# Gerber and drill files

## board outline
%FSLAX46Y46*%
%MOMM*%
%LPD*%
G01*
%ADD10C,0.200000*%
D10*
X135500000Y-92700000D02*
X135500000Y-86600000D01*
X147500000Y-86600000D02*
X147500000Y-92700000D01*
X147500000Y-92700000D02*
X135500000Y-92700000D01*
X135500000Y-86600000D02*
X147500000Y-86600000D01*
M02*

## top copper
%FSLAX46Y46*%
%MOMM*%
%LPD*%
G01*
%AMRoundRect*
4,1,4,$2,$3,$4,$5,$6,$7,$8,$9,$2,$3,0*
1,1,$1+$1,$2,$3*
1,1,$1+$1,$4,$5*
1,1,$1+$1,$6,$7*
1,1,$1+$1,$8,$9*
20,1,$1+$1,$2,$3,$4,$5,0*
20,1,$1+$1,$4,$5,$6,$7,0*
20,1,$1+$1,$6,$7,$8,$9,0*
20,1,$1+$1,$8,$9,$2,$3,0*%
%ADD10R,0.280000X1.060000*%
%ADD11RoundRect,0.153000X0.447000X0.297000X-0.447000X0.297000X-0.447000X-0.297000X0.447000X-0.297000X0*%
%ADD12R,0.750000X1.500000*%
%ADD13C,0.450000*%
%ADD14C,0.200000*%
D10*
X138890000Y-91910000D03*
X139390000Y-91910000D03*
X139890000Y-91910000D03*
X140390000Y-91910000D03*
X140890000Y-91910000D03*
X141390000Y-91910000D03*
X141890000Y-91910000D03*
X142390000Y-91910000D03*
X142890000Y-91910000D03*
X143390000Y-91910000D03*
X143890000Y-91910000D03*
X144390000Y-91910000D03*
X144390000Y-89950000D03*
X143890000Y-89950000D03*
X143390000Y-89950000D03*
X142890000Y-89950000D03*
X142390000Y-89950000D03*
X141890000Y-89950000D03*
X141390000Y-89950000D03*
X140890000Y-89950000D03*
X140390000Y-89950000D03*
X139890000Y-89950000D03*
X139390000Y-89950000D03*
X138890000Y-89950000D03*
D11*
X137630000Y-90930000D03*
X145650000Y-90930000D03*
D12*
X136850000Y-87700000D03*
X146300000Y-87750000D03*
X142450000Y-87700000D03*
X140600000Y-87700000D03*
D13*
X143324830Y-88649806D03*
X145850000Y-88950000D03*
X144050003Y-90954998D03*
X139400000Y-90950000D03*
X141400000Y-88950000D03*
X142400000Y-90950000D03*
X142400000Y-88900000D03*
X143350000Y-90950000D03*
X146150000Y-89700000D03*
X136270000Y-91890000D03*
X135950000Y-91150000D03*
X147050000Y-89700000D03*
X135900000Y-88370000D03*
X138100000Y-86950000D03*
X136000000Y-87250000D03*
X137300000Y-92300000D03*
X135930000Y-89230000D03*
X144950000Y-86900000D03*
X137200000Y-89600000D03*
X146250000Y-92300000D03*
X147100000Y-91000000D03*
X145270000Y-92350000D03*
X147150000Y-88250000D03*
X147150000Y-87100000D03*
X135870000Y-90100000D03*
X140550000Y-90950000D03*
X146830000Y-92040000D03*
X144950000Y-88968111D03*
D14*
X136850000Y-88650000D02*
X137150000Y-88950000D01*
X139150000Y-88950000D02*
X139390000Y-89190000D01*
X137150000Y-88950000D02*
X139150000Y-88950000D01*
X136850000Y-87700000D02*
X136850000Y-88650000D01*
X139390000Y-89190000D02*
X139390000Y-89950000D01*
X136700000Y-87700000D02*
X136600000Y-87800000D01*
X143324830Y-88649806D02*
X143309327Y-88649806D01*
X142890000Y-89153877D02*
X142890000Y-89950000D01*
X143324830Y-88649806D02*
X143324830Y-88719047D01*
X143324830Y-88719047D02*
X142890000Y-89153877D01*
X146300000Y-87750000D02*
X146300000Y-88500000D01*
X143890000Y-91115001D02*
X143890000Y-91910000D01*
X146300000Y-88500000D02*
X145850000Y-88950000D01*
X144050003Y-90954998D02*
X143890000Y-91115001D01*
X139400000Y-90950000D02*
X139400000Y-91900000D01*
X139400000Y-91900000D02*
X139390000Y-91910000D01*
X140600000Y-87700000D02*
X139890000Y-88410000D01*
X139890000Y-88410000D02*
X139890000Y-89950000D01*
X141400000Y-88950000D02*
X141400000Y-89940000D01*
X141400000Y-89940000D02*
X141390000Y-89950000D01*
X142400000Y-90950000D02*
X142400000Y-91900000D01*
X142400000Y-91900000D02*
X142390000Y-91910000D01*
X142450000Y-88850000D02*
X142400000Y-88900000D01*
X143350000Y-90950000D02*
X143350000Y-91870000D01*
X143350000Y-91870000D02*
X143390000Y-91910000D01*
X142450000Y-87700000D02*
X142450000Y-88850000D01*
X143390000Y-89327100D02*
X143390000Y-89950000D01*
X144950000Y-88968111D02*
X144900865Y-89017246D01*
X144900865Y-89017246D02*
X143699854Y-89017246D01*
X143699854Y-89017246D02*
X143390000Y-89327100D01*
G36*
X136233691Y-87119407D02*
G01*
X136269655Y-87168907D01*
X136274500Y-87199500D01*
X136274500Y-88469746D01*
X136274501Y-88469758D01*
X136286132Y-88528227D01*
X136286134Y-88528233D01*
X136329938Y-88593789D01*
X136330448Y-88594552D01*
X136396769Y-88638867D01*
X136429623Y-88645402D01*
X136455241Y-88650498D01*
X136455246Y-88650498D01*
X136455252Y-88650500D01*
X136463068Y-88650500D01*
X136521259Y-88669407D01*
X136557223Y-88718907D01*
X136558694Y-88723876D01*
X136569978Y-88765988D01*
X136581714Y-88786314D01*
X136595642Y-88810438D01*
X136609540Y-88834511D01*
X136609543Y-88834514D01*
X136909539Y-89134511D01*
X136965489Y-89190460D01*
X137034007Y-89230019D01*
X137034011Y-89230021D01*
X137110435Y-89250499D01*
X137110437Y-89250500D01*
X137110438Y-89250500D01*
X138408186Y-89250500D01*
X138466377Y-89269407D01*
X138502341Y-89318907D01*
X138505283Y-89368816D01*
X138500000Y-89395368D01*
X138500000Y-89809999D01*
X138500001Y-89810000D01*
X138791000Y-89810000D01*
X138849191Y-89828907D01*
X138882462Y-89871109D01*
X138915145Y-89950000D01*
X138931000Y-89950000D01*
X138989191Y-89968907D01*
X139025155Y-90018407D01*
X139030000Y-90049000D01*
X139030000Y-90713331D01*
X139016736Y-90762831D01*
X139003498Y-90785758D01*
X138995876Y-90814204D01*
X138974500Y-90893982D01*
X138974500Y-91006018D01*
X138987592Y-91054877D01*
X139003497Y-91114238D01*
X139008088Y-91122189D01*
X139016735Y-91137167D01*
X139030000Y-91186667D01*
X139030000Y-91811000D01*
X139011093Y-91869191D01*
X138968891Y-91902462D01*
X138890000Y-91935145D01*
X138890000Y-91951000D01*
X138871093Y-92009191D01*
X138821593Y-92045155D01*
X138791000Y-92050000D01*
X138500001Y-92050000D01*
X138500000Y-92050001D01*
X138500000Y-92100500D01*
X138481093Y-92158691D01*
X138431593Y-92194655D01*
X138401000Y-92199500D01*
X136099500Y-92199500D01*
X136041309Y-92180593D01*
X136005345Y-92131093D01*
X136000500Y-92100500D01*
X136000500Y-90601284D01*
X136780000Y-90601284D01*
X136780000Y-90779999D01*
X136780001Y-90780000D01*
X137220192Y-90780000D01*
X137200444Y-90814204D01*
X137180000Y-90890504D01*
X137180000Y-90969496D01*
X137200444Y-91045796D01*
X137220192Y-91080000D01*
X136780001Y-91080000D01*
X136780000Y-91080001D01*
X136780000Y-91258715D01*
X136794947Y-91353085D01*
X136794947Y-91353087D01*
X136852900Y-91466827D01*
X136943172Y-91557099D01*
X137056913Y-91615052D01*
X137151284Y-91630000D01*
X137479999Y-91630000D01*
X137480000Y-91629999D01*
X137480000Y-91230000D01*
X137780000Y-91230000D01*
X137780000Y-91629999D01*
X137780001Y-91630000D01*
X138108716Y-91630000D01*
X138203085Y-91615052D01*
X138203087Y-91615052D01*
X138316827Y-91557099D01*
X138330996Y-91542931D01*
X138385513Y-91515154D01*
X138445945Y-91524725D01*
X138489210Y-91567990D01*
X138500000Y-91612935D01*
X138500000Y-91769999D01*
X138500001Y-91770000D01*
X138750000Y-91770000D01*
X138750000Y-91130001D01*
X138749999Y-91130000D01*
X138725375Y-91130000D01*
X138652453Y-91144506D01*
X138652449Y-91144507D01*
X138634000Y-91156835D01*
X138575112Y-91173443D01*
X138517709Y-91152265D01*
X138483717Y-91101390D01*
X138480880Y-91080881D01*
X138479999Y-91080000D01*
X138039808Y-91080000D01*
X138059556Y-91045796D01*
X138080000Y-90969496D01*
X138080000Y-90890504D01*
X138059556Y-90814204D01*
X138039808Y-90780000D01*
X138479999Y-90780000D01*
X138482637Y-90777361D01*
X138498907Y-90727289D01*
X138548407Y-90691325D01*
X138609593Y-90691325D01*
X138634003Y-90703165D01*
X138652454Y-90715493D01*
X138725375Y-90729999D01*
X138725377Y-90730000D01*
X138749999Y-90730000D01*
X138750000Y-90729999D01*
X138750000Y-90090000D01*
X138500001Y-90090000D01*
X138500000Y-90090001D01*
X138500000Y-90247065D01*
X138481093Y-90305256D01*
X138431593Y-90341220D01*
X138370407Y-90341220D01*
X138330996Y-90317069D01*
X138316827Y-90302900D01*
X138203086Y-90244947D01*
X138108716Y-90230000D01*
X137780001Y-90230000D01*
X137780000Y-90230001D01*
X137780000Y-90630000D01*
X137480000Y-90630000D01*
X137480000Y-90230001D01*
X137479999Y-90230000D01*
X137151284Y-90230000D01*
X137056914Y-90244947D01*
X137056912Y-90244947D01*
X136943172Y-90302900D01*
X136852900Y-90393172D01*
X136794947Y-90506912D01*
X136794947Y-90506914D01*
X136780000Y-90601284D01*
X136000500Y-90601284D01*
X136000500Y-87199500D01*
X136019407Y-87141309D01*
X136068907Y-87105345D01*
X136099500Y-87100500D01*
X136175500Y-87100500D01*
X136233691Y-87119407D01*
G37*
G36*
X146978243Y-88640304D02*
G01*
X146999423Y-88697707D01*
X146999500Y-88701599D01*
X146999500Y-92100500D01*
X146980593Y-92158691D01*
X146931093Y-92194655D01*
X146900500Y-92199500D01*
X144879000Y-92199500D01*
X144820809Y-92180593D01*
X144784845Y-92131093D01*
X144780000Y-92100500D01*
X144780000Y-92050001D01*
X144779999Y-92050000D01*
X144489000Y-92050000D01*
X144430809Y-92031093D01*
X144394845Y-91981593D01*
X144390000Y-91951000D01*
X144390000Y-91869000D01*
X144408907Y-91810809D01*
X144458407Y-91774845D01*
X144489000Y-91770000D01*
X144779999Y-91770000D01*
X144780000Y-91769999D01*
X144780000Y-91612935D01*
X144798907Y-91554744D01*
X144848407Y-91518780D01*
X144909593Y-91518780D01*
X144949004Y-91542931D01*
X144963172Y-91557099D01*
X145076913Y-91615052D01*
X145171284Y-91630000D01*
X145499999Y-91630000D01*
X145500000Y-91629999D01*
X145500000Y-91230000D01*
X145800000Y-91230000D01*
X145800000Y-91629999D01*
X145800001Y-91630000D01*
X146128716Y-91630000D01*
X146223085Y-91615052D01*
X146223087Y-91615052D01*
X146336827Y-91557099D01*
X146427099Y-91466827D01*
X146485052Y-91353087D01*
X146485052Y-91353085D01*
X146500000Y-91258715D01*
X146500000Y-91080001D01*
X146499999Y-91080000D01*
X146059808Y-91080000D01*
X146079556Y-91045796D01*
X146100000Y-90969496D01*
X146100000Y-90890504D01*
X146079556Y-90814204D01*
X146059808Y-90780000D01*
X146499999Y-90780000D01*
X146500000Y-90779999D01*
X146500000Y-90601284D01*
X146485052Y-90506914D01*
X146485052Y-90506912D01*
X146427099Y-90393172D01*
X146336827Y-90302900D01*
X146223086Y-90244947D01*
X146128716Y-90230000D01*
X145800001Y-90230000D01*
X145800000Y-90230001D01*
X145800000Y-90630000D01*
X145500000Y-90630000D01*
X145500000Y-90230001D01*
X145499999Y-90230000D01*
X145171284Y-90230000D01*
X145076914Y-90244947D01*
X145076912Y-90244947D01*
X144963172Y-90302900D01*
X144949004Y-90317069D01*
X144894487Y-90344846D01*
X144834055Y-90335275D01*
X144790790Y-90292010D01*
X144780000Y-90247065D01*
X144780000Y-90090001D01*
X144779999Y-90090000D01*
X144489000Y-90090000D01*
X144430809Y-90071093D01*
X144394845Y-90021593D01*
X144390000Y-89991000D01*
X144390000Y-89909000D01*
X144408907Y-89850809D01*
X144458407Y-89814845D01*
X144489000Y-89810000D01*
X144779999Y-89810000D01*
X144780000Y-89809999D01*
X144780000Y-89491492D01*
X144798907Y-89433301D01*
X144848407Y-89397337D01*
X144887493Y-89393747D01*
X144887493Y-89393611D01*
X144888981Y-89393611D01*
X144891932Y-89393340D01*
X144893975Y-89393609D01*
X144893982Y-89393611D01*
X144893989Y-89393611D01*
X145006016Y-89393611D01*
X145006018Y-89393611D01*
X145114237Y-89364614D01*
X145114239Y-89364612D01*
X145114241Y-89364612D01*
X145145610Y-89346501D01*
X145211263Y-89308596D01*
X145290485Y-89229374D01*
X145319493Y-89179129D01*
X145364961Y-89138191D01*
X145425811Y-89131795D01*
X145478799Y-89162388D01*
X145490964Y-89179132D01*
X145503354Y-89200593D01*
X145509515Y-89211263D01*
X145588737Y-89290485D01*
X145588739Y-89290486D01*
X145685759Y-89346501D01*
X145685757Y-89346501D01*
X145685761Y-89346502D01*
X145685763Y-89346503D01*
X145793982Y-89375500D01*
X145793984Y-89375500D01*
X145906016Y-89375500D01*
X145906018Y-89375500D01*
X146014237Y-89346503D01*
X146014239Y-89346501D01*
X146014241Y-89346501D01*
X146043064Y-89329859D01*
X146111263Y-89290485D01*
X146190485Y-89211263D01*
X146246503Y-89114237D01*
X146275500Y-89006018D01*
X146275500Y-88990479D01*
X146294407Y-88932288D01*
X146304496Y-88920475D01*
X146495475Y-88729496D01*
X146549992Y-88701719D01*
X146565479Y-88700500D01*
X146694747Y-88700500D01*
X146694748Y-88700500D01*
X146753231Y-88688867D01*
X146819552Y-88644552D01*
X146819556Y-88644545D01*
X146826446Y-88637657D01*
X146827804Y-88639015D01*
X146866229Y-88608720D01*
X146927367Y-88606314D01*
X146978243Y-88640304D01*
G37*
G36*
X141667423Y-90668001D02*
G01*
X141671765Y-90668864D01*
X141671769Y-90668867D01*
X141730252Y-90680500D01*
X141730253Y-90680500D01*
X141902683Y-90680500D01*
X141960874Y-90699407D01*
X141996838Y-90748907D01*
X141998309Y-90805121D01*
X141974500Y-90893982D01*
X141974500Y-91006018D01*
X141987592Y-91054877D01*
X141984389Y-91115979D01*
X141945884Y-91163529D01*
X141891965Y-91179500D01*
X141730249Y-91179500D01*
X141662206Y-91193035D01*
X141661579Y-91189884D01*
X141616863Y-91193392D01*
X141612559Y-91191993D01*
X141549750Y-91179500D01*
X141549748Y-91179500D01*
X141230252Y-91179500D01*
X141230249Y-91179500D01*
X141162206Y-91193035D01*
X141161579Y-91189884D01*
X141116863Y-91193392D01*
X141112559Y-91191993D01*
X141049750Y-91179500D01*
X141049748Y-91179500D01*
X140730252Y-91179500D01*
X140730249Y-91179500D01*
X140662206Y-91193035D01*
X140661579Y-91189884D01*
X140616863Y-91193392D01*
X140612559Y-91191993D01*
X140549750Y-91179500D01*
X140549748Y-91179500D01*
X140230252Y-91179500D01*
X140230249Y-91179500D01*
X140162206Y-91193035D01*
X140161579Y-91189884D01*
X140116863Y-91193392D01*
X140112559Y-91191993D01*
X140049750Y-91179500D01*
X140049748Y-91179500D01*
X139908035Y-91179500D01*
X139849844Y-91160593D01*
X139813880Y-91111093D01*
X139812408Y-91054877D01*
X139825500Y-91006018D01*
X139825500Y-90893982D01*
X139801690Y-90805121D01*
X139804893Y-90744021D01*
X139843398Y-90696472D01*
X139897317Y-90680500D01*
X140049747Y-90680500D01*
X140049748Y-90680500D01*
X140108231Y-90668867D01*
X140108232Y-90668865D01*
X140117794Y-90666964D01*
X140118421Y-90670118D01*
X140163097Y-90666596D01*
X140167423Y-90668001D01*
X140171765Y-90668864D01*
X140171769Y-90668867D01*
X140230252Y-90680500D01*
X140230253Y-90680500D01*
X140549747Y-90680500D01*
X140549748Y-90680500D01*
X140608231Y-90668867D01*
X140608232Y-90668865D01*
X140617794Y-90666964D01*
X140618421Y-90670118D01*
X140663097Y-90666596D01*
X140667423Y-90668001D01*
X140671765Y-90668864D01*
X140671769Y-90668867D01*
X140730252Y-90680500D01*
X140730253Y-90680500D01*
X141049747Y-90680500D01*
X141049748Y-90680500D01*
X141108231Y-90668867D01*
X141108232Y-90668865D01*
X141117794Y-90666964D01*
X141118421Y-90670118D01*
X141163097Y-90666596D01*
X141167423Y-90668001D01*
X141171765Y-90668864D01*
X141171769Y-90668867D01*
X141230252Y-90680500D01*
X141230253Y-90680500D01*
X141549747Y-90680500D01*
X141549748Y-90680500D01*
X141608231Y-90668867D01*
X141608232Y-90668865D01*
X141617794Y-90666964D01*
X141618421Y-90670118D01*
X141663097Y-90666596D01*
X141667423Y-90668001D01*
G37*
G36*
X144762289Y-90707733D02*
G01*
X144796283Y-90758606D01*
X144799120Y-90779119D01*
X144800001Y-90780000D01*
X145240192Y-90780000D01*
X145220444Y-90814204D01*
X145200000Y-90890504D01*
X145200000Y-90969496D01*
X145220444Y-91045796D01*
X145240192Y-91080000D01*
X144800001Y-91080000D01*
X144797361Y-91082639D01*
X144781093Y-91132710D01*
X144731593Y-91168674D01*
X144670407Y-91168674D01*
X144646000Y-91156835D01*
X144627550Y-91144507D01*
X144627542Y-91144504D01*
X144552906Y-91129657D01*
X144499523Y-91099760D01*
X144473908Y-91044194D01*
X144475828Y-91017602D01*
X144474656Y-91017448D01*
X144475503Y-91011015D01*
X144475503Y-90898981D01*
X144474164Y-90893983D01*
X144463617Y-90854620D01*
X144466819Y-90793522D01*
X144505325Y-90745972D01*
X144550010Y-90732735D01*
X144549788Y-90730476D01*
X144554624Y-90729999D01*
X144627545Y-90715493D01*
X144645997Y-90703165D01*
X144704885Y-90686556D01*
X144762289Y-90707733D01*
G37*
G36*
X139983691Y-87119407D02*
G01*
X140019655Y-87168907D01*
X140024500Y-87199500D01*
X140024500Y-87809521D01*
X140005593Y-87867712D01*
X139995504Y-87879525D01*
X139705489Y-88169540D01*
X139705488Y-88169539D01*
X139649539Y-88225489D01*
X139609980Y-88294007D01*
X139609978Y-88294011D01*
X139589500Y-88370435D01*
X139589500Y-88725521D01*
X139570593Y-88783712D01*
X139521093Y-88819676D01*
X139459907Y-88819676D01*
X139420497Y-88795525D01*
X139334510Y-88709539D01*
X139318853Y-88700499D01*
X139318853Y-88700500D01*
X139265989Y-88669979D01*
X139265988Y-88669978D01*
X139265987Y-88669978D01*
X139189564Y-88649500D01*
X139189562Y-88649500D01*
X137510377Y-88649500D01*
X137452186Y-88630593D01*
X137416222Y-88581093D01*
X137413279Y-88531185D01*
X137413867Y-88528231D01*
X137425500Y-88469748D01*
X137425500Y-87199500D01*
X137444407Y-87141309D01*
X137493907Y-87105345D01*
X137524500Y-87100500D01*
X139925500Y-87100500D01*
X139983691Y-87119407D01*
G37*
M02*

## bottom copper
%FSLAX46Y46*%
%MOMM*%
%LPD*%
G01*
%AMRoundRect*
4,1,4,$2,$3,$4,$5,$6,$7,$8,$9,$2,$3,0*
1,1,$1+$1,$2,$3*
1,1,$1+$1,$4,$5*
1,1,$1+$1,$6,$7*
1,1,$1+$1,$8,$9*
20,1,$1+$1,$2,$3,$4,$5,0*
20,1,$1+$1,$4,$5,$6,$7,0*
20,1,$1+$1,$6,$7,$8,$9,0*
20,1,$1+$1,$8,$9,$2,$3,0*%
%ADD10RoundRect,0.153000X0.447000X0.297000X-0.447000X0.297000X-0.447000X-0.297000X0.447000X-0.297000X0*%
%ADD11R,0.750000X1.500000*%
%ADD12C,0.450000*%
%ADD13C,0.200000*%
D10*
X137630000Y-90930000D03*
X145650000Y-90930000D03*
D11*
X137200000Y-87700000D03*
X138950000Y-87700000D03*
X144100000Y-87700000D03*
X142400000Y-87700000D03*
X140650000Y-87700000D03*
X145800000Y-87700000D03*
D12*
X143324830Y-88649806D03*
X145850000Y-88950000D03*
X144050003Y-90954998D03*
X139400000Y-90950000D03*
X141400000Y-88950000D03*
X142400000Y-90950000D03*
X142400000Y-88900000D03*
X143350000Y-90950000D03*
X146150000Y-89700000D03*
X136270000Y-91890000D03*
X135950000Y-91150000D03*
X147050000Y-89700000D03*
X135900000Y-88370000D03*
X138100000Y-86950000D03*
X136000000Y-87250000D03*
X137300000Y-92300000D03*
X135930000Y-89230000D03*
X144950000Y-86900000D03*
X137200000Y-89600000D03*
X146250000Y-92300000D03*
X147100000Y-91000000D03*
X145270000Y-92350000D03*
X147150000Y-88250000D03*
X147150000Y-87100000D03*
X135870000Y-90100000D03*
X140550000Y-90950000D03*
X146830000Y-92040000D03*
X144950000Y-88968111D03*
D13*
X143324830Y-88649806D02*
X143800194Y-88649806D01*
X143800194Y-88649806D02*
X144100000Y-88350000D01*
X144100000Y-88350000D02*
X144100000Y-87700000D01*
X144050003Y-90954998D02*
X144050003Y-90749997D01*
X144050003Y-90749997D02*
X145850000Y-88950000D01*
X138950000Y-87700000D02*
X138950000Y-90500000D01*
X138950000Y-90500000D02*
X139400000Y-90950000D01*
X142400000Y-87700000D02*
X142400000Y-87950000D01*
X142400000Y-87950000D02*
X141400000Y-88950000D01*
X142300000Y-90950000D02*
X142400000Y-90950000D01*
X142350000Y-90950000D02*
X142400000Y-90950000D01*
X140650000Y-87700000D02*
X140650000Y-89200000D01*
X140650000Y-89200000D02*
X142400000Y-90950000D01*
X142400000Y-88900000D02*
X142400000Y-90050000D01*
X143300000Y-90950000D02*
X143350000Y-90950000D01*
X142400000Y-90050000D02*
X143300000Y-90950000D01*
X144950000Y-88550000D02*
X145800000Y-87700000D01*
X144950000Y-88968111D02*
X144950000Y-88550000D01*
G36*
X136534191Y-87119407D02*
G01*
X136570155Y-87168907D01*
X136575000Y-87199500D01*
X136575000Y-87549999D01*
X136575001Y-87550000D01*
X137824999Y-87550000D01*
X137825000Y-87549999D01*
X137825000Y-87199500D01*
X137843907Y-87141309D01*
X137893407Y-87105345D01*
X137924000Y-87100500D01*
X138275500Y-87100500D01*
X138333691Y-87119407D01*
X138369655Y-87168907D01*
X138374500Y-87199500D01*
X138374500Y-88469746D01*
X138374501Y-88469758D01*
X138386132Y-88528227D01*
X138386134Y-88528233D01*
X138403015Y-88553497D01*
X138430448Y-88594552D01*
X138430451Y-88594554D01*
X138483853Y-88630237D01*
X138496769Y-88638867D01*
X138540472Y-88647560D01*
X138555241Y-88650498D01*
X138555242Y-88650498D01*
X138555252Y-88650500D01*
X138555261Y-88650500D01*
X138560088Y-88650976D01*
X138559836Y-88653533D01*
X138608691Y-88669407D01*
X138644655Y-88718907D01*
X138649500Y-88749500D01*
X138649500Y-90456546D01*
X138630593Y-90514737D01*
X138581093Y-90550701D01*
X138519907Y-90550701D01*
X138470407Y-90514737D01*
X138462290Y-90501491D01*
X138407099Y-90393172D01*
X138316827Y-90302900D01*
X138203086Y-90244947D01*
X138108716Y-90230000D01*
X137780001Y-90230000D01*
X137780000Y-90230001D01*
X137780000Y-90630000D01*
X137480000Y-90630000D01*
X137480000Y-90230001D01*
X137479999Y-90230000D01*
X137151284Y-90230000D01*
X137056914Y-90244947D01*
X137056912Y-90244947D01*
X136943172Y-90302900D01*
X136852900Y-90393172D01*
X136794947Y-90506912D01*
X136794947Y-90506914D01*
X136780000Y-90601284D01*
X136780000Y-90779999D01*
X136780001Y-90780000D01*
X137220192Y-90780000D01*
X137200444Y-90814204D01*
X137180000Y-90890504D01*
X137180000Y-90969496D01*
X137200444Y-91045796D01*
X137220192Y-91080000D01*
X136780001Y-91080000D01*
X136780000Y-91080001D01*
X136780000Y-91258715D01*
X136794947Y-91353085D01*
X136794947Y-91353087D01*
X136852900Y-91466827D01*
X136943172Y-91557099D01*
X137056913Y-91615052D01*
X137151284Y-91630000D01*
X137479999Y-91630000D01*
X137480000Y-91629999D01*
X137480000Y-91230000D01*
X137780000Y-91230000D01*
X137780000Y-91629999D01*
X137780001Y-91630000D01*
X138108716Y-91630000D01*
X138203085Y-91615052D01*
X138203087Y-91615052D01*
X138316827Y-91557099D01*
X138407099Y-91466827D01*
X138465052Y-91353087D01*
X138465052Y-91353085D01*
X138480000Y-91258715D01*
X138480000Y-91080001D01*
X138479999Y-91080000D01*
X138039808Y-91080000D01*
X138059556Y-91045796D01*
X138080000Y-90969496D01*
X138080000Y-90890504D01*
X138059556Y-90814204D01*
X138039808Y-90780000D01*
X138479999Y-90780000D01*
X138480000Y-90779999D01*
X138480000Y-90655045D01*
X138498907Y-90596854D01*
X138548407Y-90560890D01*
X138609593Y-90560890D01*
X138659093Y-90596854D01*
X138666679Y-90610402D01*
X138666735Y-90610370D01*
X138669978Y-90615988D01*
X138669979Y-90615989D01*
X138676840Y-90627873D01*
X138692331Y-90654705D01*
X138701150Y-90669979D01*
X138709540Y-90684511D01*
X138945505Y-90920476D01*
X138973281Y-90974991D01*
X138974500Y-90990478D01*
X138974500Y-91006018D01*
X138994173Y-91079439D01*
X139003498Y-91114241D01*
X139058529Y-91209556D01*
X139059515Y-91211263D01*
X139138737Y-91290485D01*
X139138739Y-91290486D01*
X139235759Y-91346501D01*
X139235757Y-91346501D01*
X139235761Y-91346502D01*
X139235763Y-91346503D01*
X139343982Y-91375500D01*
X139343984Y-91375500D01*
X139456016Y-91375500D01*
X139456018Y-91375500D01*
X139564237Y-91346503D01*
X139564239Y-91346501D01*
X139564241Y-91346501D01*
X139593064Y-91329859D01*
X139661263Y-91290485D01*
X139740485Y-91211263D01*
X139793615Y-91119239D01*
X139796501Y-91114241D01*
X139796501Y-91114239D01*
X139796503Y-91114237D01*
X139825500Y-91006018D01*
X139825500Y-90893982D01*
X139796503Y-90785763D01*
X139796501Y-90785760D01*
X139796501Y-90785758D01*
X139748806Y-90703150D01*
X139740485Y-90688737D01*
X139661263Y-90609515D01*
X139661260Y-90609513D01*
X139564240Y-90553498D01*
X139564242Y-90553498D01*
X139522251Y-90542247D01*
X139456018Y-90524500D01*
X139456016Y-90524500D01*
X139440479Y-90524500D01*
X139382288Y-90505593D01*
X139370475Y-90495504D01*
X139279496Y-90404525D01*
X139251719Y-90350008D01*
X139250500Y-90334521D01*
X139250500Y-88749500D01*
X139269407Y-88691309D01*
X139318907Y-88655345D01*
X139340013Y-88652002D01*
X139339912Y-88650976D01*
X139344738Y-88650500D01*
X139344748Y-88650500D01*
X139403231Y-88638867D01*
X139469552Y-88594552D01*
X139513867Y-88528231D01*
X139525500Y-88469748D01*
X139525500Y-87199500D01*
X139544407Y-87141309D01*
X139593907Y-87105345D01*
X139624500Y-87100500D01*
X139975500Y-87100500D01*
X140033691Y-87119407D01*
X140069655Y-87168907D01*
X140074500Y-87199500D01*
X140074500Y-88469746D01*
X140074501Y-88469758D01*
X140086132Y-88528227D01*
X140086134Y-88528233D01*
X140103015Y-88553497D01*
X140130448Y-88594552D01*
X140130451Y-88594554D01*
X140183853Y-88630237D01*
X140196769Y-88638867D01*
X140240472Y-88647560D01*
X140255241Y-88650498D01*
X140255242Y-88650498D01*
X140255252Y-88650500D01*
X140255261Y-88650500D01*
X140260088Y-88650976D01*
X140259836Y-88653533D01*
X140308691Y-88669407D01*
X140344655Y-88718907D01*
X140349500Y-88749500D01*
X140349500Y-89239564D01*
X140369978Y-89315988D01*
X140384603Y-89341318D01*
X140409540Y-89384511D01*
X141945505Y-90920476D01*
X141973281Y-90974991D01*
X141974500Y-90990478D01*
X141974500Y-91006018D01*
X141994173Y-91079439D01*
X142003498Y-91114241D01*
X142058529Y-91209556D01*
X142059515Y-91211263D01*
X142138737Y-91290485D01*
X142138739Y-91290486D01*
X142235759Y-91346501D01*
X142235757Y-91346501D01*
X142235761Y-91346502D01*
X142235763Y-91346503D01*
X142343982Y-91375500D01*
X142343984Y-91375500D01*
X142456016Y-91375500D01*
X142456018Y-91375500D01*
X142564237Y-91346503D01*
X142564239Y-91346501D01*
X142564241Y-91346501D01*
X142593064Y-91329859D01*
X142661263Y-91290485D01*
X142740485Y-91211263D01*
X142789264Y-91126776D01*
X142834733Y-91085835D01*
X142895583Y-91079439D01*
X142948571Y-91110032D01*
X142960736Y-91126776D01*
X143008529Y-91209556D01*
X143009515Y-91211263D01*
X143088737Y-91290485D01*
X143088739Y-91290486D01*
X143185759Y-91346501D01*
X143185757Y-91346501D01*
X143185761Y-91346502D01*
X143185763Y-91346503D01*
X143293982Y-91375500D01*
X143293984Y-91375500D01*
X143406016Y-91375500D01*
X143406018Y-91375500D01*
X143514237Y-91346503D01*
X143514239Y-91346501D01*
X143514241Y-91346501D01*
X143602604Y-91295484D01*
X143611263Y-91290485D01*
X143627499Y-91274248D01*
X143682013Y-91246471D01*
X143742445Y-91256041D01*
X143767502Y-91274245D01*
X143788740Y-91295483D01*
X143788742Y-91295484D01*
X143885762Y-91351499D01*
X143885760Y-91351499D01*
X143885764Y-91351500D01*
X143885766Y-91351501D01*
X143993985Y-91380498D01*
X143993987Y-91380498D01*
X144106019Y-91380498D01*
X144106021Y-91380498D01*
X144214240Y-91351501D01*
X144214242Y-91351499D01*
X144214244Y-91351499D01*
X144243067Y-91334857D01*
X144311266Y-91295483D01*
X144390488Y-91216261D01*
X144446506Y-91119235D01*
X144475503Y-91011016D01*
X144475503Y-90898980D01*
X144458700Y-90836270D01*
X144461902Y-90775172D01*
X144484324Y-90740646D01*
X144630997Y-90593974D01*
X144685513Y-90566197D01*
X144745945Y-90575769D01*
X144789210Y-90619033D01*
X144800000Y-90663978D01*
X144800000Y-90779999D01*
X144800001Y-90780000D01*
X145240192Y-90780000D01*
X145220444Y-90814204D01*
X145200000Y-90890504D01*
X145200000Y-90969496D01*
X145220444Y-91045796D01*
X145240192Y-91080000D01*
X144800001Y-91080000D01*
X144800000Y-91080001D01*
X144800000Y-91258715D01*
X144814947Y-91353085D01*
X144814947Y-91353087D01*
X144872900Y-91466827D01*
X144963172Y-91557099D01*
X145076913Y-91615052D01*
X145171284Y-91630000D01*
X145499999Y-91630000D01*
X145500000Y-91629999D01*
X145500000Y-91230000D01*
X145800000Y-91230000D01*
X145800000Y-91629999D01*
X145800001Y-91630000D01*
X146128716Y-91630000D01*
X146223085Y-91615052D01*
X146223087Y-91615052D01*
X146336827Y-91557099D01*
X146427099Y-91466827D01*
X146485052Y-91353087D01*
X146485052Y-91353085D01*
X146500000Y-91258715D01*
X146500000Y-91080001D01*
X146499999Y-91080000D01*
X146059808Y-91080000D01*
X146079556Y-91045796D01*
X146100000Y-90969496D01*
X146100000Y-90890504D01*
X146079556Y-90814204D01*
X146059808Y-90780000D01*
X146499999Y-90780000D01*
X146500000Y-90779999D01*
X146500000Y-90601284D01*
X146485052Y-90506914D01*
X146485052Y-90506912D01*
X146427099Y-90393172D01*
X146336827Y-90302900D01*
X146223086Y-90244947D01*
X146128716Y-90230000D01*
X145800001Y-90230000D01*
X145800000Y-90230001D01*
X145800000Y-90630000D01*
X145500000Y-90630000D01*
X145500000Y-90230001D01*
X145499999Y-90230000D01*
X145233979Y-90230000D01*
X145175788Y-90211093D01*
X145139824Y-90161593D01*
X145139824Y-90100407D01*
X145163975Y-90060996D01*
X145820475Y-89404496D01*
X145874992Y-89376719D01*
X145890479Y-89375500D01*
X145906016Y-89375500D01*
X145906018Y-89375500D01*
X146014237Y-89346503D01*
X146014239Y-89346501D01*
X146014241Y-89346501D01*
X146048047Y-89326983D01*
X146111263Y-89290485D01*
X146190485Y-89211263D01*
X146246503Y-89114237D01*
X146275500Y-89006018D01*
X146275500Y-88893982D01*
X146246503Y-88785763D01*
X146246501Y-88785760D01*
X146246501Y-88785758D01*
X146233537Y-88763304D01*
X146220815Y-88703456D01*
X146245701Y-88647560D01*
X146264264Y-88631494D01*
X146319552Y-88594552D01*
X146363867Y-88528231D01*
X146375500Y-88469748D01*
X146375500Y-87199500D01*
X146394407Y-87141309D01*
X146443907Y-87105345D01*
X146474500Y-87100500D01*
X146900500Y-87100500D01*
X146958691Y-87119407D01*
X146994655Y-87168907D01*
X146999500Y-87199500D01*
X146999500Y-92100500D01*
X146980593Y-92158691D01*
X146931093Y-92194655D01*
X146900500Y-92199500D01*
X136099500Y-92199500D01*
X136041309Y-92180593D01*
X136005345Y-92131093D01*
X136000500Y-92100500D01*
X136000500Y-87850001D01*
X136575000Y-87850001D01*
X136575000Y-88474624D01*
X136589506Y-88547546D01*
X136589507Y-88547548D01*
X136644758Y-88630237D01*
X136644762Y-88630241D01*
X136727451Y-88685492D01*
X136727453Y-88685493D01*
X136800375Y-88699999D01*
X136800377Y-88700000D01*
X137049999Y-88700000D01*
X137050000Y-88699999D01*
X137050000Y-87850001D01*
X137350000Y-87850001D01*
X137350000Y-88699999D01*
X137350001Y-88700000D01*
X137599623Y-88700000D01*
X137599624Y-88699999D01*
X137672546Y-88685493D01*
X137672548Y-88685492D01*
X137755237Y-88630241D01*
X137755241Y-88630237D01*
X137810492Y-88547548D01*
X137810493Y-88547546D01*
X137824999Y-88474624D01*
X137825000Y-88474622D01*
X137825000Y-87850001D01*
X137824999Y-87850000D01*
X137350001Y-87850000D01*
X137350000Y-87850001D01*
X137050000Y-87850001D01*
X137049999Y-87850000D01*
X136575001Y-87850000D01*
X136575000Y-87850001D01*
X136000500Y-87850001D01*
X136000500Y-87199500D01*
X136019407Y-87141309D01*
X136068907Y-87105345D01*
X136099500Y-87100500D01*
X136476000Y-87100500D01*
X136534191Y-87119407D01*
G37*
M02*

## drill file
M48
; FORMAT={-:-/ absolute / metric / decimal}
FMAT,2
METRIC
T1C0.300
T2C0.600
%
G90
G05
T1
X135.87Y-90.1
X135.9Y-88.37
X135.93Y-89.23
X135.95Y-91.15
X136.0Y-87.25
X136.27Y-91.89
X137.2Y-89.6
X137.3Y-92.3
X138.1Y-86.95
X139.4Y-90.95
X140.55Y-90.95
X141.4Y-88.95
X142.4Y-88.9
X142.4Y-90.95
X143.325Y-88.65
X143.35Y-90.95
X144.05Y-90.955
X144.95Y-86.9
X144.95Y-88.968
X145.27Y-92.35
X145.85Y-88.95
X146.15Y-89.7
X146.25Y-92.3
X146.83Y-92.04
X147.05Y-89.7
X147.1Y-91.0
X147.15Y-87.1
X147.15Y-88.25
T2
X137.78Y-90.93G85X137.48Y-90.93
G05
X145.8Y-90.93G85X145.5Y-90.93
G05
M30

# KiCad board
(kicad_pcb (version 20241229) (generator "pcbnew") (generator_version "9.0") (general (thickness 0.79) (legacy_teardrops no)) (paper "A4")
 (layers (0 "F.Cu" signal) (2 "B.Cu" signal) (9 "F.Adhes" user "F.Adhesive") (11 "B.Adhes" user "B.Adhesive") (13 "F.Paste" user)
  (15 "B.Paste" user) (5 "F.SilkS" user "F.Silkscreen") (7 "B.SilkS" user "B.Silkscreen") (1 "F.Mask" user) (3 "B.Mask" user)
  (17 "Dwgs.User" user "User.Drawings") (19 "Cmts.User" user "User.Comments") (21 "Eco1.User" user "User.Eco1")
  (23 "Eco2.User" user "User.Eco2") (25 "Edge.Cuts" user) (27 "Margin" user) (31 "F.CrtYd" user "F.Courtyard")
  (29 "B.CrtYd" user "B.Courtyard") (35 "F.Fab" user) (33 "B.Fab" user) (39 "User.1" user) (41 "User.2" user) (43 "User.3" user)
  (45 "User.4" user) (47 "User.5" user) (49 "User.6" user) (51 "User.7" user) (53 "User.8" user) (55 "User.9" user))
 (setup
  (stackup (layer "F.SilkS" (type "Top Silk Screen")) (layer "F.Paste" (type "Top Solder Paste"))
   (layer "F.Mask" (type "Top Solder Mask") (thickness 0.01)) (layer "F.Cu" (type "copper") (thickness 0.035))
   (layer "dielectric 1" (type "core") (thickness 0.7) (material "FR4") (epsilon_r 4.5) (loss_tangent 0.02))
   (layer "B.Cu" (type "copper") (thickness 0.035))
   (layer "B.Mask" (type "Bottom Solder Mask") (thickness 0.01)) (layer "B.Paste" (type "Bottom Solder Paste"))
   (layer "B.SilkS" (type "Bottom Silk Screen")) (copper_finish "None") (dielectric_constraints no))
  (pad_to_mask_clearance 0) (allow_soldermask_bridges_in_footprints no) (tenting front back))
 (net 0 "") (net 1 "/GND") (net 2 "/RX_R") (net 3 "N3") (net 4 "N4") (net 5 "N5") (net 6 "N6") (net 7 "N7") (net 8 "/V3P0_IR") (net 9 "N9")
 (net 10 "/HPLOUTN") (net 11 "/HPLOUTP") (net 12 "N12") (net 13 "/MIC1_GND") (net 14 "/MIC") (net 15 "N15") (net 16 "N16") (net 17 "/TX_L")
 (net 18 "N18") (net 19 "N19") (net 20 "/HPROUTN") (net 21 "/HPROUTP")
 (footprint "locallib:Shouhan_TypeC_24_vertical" (layer "F.Cu") (at 141.64 90.83 180)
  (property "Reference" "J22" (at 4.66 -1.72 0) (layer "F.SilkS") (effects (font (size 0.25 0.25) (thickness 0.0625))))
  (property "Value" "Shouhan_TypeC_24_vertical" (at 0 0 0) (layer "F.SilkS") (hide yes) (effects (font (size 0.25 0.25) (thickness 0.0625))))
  (pad "A1" smd rect (at 2.75 -1.08 180) (size 0.28 1.06) (layers "F.Cu" "F.Mask" "F.Paste") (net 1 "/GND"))
  (pad "A2" smd rect (at 2.25 -1.08 180) (size 0.28 1.06) (layers "F.Cu" "F.Mask" "F.Paste") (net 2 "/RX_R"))
  (pad "A3" smd rect (at 1.75 -1.08 180) (size 0.28 1.06) (layers "F.Cu" "F.Mask" "F.Paste") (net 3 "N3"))
  (pad "A4" smd rect (at 1.25 -1.08 180) (size 0.28 1.06) (layers "F.Cu" "F.Mask" "F.Paste") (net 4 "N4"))
  (pad "A5" smd rect (at 0.75 -1.08 180) (size 0.28 1.06) (layers "F.Cu" "F.Mask" "F.Paste") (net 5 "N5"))
  (pad "A6" smd rect (at 0.25 -1.08 180) (size 0.28 1.06) (layers "F.Cu" "F.Mask" "F.Paste") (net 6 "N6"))
  (pad "A7" smd rect (at -0.25 -1.08 180) (size 0.28 1.06) (layers "F.Cu" "F.Mask" "F.Paste") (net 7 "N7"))
  (pad "A8" smd rect (at -0.75 -1.08 180) (size 0.28 1.06) (layers "F.Cu" "F.Mask" "F.Paste") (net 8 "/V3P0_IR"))
  (pad "A9" smd rect (at -1.25 -1.08 180) (size 0.28 1.06) (layers "F.Cu" "F.Mask" "F.Paste") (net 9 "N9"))
  (pad "A10" smd rect (at -1.75 -1.08 180) (size 0.28 1.06) (layers "F.Cu" "F.Mask" "F.Paste") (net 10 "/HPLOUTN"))
  (pad "A11" smd rect (at -2.25 -1.08 180) (size 0.28 1.06) (layers "F.Cu" "F.Mask" "F.Paste") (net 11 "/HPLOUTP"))
  (pad "A12" smd rect (at -2.75 -1.08 180) (size 0.28 1.06) (layers "F.Cu" "F.Mask" "F.Paste") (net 1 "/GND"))
  (pad "B1" smd rect (at -2.75 0.88 180) (size 0.28 1.06) (layers "F.Cu" "F.Mask" "F.Paste") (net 1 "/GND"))
  (pad "B2" smd rect (at -2.25 0.88 180) (size 0.28 1.06) (layers "F.Cu" "F.Mask" "F.Paste") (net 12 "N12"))
  (pad "B3" smd rect (at -1.75 0.88 180) (size 0.28 1.06) (layers "F.Cu" "F.Mask" "F.Paste") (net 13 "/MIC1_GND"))
  (pad "B4" smd rect (at -1.25 0.88 180) (size 0.28 1.06) (layers "F.Cu" "F.Mask" "F.Paste") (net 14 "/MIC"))
  (pad "B5" smd rect (at -0.75 0.88 180) (size 0.28 1.06) (layers "F.Cu" "F.Mask" "F.Paste") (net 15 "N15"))
  (pad "B6" smd rect (at -0.25 0.88 180) (size 0.28 1.06) (layers "F.Cu" "F.Mask" "F.Paste") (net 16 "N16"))
  (pad "B7" smd rect (at 0.25 0.88 180) (size 0.28 1.06) (layers "F.Cu" "F.Mask" "F.Paste") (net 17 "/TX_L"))
  (pad "B8" smd rect (at 0.75 0.88 180) (size 0.28 1.06) (layers "F.Cu" "F.Mask" "F.Paste") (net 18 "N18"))
  (pad "B9" smd rect (at 1.25 0.88 180) (size 0.28 1.06) (layers "F.Cu" "F.Mask" "F.Paste") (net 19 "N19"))
  (pad "B10" smd rect (at 1.75 0.88 180) (size 0.28 1.06) (layers "F.Cu" "F.Mask" "F.Paste") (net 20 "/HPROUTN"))
  (pad "B11" smd rect (at 2.25 0.88 180) (size 0.28 1.06) (layers "F.Cu" "F.Mask" "F.Paste") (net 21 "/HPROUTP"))
  (pad "B12" smd rect (at 2.75 0.88 180) (size 0.28 1.06) (layers "F.Cu" "F.Mask" "F.Paste") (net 1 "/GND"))
  (pad "MH1" thru_hole roundrect (at 4.01 -0.1 180) (size 1.2 0.9) (drill oval 0.9 0.6) (layers "*.Cu" "*.Mask") (remove_unused_layers no)
   (roundrect_rratio 0.17) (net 1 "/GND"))
  (pad "MH2" thru_hole roundrect (at -4.01 -0.1 180) (size 1.2 0.9) (drill oval 0.9 0.6) (layers "*.Cu" "*.Mask") (remove_unused_layers no)
   (roundrect_rratio 0.17) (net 1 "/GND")))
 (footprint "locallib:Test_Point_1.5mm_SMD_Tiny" (layer "F.Cu") (at 136.85 87.7)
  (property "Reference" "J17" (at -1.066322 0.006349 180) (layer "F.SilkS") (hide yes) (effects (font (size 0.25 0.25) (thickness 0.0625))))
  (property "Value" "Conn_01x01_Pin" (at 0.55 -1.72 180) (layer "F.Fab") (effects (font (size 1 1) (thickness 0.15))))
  (pad "1" smd rect (at 0 0) (size 0.75 1.5) (layers "F.Cu" "F.Mask") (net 21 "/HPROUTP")))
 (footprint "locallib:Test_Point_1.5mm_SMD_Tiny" (layer "F.Cu") (at 146.3 87.75)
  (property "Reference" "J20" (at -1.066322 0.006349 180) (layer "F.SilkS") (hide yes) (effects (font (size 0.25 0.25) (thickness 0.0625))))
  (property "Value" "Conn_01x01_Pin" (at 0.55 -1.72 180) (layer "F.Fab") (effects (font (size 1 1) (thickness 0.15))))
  (pad "1" smd rect (at 0 0) (size 0.75 1.5) (layers "F.Cu" "F.Mask") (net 11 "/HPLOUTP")))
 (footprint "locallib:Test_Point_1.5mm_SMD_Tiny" (layer "F.Cu") (at 142.45 87.7)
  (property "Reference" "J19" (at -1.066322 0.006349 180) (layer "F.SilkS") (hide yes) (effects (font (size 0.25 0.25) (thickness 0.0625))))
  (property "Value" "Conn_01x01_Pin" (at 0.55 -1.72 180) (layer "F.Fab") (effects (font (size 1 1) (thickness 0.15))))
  (pad "1" smd rect (at 0 0) (size 0.75 1.5) (layers "F.Cu" "F.Mask") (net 10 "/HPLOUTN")))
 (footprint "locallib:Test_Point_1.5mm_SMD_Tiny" (layer "F.Cu") (at 140.6 87.7)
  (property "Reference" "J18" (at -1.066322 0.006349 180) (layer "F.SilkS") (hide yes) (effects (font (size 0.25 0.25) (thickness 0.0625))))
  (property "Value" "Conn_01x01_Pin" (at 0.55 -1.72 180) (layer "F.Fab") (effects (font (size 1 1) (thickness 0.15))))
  (pad "1" smd rect (at 0 0) (size 0.75 1.5) (layers "F.Cu" "F.Mask") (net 20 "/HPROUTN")))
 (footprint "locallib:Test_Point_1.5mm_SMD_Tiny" (layer "B.Cu") (at 137.2 87.7 180)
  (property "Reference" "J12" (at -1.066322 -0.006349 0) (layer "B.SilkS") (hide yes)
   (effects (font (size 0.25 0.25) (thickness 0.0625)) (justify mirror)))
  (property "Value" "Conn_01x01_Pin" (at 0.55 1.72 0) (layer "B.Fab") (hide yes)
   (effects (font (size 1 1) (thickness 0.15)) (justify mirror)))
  (pad "1" smd rect (at 0 0 180) (size 0.75 1.5) (layers "B.Cu" "B.Mask") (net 1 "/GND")))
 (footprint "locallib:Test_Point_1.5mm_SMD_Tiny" (layer "B.Cu") (at 138.95 87.7 180)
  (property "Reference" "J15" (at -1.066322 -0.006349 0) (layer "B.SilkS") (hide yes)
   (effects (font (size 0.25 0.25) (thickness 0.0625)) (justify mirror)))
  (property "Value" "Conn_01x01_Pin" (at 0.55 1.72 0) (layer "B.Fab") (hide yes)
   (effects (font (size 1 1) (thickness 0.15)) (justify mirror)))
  (pad "1" smd rect (at 0 0 180) (size 0.75 1.5) (layers "B.Cu" "B.Mask") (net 2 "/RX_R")))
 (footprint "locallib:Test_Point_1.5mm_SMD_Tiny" (layer "B.Cu") (at 144.1 87.7 180)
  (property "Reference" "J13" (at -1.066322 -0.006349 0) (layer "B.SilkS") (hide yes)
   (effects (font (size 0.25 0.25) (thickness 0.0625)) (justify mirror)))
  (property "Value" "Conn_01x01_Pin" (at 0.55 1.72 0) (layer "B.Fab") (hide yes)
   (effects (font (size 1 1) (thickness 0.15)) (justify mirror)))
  (pad "1" smd rect (at 0 0 180) (size 0.75 1.5) (layers "B.Cu" "B.Mask") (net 14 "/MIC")))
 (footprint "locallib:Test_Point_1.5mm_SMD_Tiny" (layer "B.Cu") (at 142.4 87.7 180)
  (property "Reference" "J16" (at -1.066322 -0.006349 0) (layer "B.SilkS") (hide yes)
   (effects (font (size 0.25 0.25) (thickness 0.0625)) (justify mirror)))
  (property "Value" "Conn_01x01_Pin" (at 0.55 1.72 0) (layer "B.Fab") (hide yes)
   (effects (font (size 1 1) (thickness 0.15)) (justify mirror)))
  (pad "1" smd rect (at 0 0 180) (size 0.75 1.5) (layers "B.Cu" "B.Mask") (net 17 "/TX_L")))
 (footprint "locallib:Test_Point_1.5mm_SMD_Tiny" (layer "B.Cu") (at 140.65 87.7 180)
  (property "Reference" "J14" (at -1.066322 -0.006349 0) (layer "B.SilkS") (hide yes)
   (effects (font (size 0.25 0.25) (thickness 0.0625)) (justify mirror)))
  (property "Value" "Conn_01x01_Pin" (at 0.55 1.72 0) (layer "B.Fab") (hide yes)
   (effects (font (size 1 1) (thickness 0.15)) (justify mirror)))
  (pad "1" smd rect (at 0 0 180) (size 0.75 1.5) (layers "B.Cu" "B.Mask") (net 8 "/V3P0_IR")))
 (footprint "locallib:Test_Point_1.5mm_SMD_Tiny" (layer "B.Cu") (at 145.8 87.7 180)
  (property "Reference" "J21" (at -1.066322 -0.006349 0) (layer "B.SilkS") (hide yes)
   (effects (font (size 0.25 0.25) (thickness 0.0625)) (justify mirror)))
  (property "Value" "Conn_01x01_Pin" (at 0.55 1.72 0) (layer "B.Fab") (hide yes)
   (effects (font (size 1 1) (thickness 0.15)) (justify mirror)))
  (pad "1" smd rect (at 0 0 180) (size 0.75 1.5) (layers "B.Cu" "B.Mask") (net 13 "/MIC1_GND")))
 (gr_line (start 135.5 92.7) (end 135.5 86.6) (stroke (width 0.2) (type solid)) (locked yes) (layer "Edge.Cuts"))
 (gr_line (start 147.5 86.6) (end 147.5 92.7) (stroke (width 0.2) (type solid)) (locked yes) (layer "Edge.Cuts"))
 (gr_line (start 147.5 92.7) (end 135.5 92.7) (stroke (width 0.2) (type solid)) (locked yes) (layer "Edge.Cuts"))
 (gr_line (start 135.5 86.6) (end 147.5 86.6) (stroke (width 0.2) (type solid)) (locked yes) (layer "Edge.Cuts"))
 (segment (start 136.85 88.65) (end 137.15 88.95) (width 0.2) (layer "F.Cu") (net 21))
 (segment (start 139.15 88.95) (end 139.39 89.19) (width 0.2) (layer "F.Cu") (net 21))
 (segment (start 137.15 88.95) (end 139.15 88.95) (width 0.2) (layer "F.Cu") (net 21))
 (segment (start 136.85 87.7) (end 136.85 88.65) (width 0.2) (layer "F.Cu") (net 21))
 (segment (start 139.39 89.19) (end 139.39 89.95) (width 0.2) (layer "F.Cu") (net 21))
 (segment (start 136.7 87.7) (end 136.6 87.8) (width 0.2) (layer "F.Cu") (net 21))
 (segment (start 143.32483 88.649806) (end 143.309327 88.649806) (width 0.2) (layer "F.Cu") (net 14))
 (segment (start 142.89 89.153877) (end 142.89 89.95) (width 0.2) (layer "F.Cu") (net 14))
 (segment (start 143.32483 88.649806) (end 143.32483 88.719047) (width 0.2) (layer "F.Cu") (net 14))
 (segment (start 143.32483 88.719047) (end 142.89 89.153877) (width 0.2) (layer "F.Cu") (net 14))
 (via (at 143.32483 88.649806) (size 0.45) (drill 0.3) (layers "F.Cu" "B.Cu") (free yes) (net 14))
 (segment (start 143.32483 88.649806) (end 143.800194 88.649806) (width 0.2) (layer "B.Cu") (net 14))
 (segment (start 143.800194 88.649806) (end 144.1 88.35) (width 0.2) (layer "B.Cu") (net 14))
 (segment (start 144.1 88.35) (end 144.1 87.7) (width 0.2) (layer "B.Cu") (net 14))
 (segment (start 146.3 87.75) (end 146.3 88.5) (width 0.2) (layer "F.Cu") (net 11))
 (segment (start 143.89 91.115001) (end 143.89 91.91) (width 0.2) (layer "F.Cu") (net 11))
 (segment (start 146.3 88.5) (end 145.85 88.95) (width 0.2) (layer "F.Cu") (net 11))
 (segment (start 144.050003 90.954998) (end 143.89 91.115001) (width 0.2) (layer "F.Cu") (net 11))
 (via (at 145.85 88.95) (size 0.45) (drill 0.3) (layers "F.Cu" "B.Cu") (free yes) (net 11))
 (via (at 144.050003 90.954998) (size 0.45) (drill 0.3) (layers "F.Cu" "B.Cu") (free yes) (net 11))
 (segment (start 144.050003 90.954998) (end 144.050003 90.749997) (width 0.2) (layer "B.Cu") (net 11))
 (segment (start 144.050003 90.749997) (end 145.85 88.95) (width 0.2) (layer "B.Cu") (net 11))
 (segment (start 139.4 90.95) (end 139.4 91.9) (width 0.2) (layer "F.Cu") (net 2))
 (segment (start 139.4 91.9) (end 139.39 91.91) (width 0.2) (layer "F.Cu") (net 2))
 (via (at 139.4 90.95) (size 0.45) (drill 0.3) (layers "F.Cu" "B.Cu") (free yes) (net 2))
 (segment (start 138.95 87.7) (end 138.95 90.5) (width 0.2) (layer "B.Cu") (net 2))
 (segment (start 138.95 90.5) (end 139.4 90.95) (width 0.2) (layer "B.Cu") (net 2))
 (segment (start 140.6 87.7) (end 139.89 88.41) (width 0.2) (layer "F.Cu") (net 20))
 (segment (start 139.89 88.41) (end 139.89 89.95) (width 0.2) (layer "F.Cu") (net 20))
 (segment (start 141.4 88.95) (end 141.4 89.94) (width 0.2) (layer "F.Cu") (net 17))
 (segment (start 141.4 89.94) (end 141.39 89.95) (width 0.2) (layer "F.Cu") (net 17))
 (via (at 141.4 88.95) (size 0.45) (drill 0.3) (layers "F.Cu" "B.Cu") (free yes) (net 17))
 (segment (start 142.4 87.7) (end 142.4 87.95) (width 0.2) (layer "B.Cu") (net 17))
 (segment (start 142.4 87.95) (end 141.4 88.95) (width 0.2) (layer "B.Cu") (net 17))
 (segment (start 142.4 90.95) (end 142.4 91.9) (width 0.2) (layer "F.Cu") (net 8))
 (segment (start 142.4 91.9) (end 142.39 91.91) (width 0.2) (layer "F.Cu") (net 8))
 (via (at 142.4 90.95) (size 0.45) (drill 0.3) (layers "F.Cu" "B.Cu") (free yes) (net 8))
 (segment (start 142.3 90.95) (end 142.4 90.95) (width 0.2) (layer "B.Cu") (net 8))
 (segment (start 142.35 90.95) (end 142.4 90.95) (width 0.2) (layer "B.Cu") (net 8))
 (segment (start 140.65 87.7) (end 140.65 89.2) (width 0.2) (layer "B.Cu") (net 8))
 (segment (start 140.65 89.2) (end 142.4 90.95) (width 0.2) (layer "B.Cu") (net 8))
 (segment (start 142.45 88.85) (end 142.4 88.9) (width 0.2) (layer "F.Cu") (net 10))
 (segment (start 143.35 90.95) (end 143.35 91.87) (width 0.2) (layer "F.Cu") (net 10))
 (segment (start 143.35 91.87) (end 143.39 91.91) (width 0.2) (layer "F.Cu") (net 10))
 (segment (start 142.45 87.7) (end 142.45 88.85) (width 0.2) (layer "F.Cu") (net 10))
 (via (at 142.4 88.9) (size 0.45) (drill 0.3) (layers "F.Cu" "B.Cu") (free yes) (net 10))
 (via (at 143.35 90.95) (size 0.45) (drill 0.3) (layers "F.Cu" "B.Cu") (free yes) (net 10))
 (segment (start 142.4 88.9) (end 142.4 90.05) (width 0.2) (layer "B.Cu") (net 10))
 (segment (start 143.3 90.95) (end 143.35 90.95) (width 0.2) (layer "B.Cu") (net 10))
 (segment (start 142.4 90.05) (end 143.3 90.95) (width 0.2) (layer "B.Cu") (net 10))
 (via (at 146.15 89.7) (size 0.45) (drill 0.3) (layers "F.Cu" "B.Cu") (free yes) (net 1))
 (via (at 136.27 91.89) (size 0.45) (drill 0.3) (layers "F.Cu" "B.Cu") (free yes) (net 1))
 (via (at 135.95 91.15) (size 0.45) (drill 0.3) (layers "F.Cu" "B.Cu") (free yes) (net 1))
 (via (at 147.05 89.7) (size 0.45) (drill 0.3) (layers "F.Cu" "B.Cu") (free yes) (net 1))
 (via (at 135.9 88.37) (size 0.45) (drill 0.3) (layers "F.Cu" "B.Cu") (free yes) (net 1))
 (via (at 138.1 86.95) (size 0.45) (drill 0.3) (layers "F.Cu" "B.Cu") (free yes) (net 1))
 (via (at 136 87.25) (size 0.45) (drill 0.3) (layers "F.Cu" "B.Cu") (free yes) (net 1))
 (via (at 137.3 92.3) (size 0.45) (drill 0.3) (layers "F.Cu" "B.Cu") (free yes) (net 1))
 (via (at 135.93 89.23) (size 0.45) (drill 0.3) (layers "F.Cu" "B.Cu") (free yes) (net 1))
 (via (at 144.95 86.9) (size 0.45) (drill 0.3) (layers "F.Cu" "B.Cu") (free yes) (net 1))
 (via (at 137.2 89.6) (size 0.45) (drill 0.3) (layers "F.Cu" "B.Cu") (free yes) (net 1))
 (via (at 146.25 92.3) (size 0.45) (drill 0.3) (layers "F.Cu" "B.Cu") (free yes) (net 1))
 (via (at 147.1 91) (size 0.45) (drill 0.3) (layers "F.Cu" "B.Cu") (free yes) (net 1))
 (via (at 145.27 92.35) (size 0.45) (drill 0.3) (layers "F.Cu" "B.Cu") (free yes) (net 1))
 (via (at 147.15 88.25) (size 0.45) (drill 0.3) (layers "F.Cu" "B.Cu") (free yes) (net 1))
 (via (at 147.15 87.1) (size 0.45) (drill 0.3) (layers "F.Cu" "B.Cu") (free yes) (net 1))
 (via (at 135.87 90.1) (size 0.45) (drill 0.3) (layers "F.Cu" "B.Cu") (free yes) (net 1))
 (via (at 140.55 90.95) (size 0.45) (drill 0.3) (layers "F.Cu" "B.Cu") (free yes) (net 1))
 (via (at 146.83 92.04) (size 0.45) (drill 0.3) (layers "F.Cu" "B.Cu") (free yes) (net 1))
 (segment (start 143.39 89.3271) (end 143.39 89.95) (width 0.2) (layer "F.Cu") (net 13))
 (segment (start 144.95 88.968111) (end 144.900865 89.017246) (width 0.2) (layer "F.Cu") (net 13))
 (segment (start 144.900865 89.017246) (end 143.699854 89.017246) (width 0.2) (layer "F.Cu") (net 13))
 (segment (start 143.699854 89.017246) (end 143.39 89.3271) (width 0.2) (layer "F.Cu") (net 13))
 (via (at 144.95 88.968111) (size 0.45) (drill 0.3) (layers "F.Cu" "B.Cu") (free yes) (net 13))
 (segment (start 144.95 88.55) (end 145.8 87.7) (width 0.2) (layer "B.Cu") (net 13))
 (segment (start 144.95 88.968111) (end 144.95 88.55) (width 0.2) (layer "B.Cu") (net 13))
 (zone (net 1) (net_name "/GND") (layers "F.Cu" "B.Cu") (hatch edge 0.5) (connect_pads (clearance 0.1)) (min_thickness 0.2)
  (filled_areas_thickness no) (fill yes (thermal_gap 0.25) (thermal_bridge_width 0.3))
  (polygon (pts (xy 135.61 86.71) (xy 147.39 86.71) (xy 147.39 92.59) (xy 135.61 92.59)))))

